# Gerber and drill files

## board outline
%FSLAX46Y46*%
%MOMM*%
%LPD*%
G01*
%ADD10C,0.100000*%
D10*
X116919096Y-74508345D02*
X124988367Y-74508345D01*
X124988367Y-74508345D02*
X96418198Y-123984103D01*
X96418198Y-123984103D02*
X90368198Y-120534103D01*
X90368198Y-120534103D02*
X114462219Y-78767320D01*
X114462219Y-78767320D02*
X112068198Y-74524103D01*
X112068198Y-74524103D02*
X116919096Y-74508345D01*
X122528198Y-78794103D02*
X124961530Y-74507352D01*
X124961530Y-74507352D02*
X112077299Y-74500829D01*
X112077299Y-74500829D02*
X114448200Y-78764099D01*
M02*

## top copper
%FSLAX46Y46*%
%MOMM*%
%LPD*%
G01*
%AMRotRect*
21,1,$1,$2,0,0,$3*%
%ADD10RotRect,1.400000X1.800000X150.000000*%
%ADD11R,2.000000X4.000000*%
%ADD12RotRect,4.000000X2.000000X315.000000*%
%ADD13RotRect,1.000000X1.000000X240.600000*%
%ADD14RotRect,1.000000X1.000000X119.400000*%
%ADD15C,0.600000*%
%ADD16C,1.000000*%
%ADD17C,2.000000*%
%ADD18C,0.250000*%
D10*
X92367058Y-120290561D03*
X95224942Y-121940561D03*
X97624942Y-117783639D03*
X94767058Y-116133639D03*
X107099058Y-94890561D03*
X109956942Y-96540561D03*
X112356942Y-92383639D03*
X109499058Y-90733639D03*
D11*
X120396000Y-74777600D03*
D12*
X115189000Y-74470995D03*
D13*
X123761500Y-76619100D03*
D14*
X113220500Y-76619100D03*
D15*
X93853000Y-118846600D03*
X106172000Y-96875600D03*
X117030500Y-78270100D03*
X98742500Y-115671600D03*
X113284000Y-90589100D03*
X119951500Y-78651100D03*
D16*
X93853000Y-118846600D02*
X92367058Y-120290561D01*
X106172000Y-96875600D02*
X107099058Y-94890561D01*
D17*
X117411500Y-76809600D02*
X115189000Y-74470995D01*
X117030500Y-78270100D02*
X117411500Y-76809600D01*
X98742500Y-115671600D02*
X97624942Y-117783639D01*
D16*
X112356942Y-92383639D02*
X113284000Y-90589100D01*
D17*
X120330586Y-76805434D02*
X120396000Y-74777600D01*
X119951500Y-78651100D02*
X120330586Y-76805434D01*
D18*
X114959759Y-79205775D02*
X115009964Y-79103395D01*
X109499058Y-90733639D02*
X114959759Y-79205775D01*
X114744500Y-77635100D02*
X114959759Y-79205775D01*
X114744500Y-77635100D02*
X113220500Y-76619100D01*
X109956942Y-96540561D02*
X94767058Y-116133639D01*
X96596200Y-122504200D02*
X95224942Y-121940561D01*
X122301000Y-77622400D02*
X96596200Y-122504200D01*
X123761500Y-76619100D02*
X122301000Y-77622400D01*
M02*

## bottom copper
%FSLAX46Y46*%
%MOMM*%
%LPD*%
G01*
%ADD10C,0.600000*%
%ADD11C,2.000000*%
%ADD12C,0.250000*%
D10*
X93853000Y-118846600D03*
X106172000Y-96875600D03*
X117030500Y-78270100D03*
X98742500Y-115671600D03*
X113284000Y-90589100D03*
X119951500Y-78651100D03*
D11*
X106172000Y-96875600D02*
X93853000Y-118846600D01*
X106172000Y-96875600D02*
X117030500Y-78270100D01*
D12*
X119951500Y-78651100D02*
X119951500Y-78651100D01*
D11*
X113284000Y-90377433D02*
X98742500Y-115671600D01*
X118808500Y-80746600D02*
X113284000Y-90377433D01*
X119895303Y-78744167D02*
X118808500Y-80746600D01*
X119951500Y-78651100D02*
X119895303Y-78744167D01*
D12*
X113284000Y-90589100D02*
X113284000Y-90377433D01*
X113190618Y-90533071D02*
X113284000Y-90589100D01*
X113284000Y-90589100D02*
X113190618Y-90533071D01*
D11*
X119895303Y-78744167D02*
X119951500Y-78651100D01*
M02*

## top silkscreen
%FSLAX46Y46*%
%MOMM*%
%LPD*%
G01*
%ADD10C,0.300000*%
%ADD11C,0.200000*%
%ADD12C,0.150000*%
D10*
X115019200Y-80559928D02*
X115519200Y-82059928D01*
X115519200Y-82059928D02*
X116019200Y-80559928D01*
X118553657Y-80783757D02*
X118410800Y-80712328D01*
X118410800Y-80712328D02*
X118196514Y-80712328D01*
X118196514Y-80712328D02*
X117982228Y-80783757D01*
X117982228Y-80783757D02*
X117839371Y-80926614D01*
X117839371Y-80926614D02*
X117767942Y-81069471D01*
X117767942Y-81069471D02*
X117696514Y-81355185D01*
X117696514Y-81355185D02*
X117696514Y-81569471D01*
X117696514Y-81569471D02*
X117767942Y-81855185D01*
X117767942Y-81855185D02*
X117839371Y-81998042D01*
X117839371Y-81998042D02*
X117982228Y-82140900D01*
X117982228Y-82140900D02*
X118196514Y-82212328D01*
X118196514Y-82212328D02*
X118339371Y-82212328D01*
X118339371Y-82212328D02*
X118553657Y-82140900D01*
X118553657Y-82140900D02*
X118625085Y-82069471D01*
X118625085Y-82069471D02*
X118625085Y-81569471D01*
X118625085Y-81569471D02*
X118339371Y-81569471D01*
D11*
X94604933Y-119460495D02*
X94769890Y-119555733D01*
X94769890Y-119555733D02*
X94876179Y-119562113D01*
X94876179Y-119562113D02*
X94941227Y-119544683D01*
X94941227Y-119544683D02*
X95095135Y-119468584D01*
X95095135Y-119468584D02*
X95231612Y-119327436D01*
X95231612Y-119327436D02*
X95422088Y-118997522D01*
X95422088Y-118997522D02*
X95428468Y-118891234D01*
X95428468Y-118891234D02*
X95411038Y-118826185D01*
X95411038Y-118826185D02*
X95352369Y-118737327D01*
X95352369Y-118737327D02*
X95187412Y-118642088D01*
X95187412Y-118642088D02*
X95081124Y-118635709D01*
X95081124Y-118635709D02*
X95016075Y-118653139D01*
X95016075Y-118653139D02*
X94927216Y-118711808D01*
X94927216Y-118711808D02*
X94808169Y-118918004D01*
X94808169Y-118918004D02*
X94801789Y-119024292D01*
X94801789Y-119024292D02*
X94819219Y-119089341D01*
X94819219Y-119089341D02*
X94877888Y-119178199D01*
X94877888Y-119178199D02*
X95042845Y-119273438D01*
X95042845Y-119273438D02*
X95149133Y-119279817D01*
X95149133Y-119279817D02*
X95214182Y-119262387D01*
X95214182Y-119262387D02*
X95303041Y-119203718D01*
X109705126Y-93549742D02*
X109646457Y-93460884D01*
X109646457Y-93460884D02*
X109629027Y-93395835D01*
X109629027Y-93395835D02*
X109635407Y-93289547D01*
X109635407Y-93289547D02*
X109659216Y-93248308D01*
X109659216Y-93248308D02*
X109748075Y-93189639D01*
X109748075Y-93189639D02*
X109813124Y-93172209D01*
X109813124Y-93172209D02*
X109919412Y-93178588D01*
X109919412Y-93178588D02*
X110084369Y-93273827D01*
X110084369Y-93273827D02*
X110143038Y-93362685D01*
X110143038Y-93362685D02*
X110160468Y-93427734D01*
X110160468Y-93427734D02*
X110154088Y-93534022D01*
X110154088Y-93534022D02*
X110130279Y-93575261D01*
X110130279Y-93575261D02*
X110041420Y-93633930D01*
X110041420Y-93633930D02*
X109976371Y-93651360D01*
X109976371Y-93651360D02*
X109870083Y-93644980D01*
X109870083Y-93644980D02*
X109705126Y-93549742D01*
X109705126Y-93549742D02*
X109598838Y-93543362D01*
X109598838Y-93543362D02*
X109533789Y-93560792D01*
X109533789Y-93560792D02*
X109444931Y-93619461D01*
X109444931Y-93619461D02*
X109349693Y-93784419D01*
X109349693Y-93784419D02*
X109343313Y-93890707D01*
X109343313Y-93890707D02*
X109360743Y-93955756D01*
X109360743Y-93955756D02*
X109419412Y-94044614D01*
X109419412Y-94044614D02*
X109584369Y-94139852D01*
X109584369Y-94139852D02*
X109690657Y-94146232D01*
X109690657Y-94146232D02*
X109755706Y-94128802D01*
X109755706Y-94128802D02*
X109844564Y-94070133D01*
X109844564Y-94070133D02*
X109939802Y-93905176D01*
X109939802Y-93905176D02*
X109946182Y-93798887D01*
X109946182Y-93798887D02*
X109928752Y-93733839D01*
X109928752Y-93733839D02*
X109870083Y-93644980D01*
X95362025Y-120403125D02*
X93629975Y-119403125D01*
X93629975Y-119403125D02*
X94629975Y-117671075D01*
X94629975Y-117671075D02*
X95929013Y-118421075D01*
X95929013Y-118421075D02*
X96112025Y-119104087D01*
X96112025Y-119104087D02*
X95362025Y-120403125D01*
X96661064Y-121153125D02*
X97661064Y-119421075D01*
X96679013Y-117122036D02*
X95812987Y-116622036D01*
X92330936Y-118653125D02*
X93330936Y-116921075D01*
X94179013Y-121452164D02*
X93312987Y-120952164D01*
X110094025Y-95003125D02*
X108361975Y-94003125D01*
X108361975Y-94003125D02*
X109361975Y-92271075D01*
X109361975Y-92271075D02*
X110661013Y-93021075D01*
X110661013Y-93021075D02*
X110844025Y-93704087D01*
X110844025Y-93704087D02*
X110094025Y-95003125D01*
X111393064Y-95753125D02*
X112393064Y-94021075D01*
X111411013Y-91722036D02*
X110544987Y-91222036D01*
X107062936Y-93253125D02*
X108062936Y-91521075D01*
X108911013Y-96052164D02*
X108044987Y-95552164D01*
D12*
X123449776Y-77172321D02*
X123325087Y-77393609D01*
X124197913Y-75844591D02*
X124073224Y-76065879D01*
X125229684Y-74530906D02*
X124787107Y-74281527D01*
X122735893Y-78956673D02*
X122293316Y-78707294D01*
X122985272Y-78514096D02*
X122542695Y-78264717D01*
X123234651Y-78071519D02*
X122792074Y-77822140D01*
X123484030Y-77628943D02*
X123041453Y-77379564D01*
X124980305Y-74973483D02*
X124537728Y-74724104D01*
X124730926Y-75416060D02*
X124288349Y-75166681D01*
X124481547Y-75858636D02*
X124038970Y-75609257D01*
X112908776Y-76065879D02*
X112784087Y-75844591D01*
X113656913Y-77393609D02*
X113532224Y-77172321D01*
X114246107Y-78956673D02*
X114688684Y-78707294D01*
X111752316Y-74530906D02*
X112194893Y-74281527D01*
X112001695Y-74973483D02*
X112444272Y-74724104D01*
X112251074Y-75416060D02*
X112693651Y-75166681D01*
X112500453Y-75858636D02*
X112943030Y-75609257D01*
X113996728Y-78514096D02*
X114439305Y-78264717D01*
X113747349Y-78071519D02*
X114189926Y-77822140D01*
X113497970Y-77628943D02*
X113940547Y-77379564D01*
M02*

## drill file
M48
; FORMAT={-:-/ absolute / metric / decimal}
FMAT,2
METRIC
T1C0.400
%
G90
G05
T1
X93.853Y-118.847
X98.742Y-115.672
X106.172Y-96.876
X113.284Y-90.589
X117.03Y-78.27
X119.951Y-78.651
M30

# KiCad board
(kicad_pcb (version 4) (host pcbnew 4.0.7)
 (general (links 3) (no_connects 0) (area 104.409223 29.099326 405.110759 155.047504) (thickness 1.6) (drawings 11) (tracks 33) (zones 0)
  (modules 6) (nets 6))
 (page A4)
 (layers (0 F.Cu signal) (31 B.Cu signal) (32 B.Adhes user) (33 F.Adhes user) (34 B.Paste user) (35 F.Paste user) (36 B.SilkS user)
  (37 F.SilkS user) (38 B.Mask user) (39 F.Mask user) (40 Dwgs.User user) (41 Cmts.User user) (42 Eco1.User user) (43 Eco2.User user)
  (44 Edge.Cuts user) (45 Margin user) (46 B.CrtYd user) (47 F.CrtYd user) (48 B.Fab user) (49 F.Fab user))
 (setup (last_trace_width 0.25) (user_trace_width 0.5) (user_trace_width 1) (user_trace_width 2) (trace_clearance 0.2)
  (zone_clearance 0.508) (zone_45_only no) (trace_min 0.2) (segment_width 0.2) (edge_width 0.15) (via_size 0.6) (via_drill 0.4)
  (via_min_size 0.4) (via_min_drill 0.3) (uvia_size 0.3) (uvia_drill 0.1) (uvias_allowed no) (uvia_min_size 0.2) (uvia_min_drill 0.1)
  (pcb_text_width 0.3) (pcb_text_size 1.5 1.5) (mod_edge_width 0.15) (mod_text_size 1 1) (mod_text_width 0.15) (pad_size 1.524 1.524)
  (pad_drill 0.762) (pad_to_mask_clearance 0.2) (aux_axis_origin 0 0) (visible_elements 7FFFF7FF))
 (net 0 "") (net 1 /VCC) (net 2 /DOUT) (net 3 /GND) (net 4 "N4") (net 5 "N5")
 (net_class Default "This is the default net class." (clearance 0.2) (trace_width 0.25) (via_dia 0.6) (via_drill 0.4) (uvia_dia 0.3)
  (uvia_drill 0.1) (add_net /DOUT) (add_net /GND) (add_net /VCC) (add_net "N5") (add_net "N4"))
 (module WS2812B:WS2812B (layer F.Cu) (at 94.996 119.0371 150)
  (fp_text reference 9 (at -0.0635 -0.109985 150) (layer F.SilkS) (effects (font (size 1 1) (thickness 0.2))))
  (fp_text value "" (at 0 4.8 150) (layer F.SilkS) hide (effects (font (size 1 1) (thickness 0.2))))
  (fp_line (start -1 -1) (end 1 -1) (layer F.SilkS) (width 0.2)) (fp_line (start 1 -1) (end 1 1) (layer F.SilkS) (width 0.2))
  (fp_line (start 1 1) (end -0.5 1) (layer F.SilkS) (width 0.2))
  (fp_line (start -0.5 1) (end -1 0.5) (layer F.SilkS) (width 0.2))
  (fp_line (start -1 0.5) (end -1 -1) (layer F.SilkS) (width 0.2))
  (fp_line (start -2.5 -1) (end -2.5 1) (layer F.SilkS) (width 0.2))
  (fp_line (start -0.5 2.5) (end 0.5 2.5) (layer F.SilkS) (width 0.2))
  (fp_line (start 2.5 -1) (end 2.5 1) (layer F.SilkS) (width 0.2))
  (fp_line (start -0.5 -2.5) (end 0.5 -2.5) (layer F.SilkS) (width 0.2))
  (pad 1 smd rect (at 1.65 -2.4 150) (size 1.4 1.8) (layers F.Cu F.Paste F.Mask) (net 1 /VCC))
  (pad 2 smd rect (at -1.65 -2.4 150) (size 1.4 1.8) (layers F.Cu F.Paste F.Mask) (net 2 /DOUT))
  (pad 3 smd rect (at -1.65 2.4 150) (size 1.4 1.8) (layers F.Cu F.Paste F.Mask) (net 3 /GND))
  (pad 4 smd rect (at 1.65 2.4 150) (size 1.4 1.8) (layers F.Cu F.Paste F.Mask) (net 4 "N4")))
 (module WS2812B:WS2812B (layer F.Cu) (at 109.728 93.6371 150)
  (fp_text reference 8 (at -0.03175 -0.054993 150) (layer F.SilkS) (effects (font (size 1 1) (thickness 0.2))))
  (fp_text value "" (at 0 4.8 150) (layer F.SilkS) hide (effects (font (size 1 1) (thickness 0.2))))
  (fp_line (start -1 -1) (end 1 -1) (layer F.SilkS) (width 0.2)) (fp_line (start 1 -1) (end 1 1) (layer F.SilkS) (width 0.2))
  (fp_line (start 1 1) (end -0.5 1) (layer F.SilkS) (width 0.2))
  (fp_line (start -0.5 1) (end -1 0.5) (layer F.SilkS) (width 0.2))
  (fp_line (start -1 0.5) (end -1 -1) (layer F.SilkS) (width 0.2))
  (fp_line (start -2.5 -1) (end -2.5 1) (layer F.SilkS) (width 0.2))
  (fp_line (start -0.5 2.5) (end 0.5 2.5) (layer F.SilkS) (width 0.2))
  (fp_line (start 2.5 -1) (end 2.5 1) (layer F.SilkS) (width 0.2))
  (fp_line (start -0.5 -2.5) (end 0.5 -2.5) (layer F.SilkS) (width 0.2))
  (pad 1 smd rect (at 1.65 -2.4 150) (size 1.4 1.8) (layers F.Cu F.Paste F.Mask) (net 1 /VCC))
  (pad 2 smd rect (at -1.65 -2.4 150) (size 1.4 1.8) (layers F.Cu F.Paste F.Mask) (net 4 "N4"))
  (pad 3 smd rect (at -1.65 2.4 150) (size 1.4 1.8) (layers F.Cu F.Paste F.Mask) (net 3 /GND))
  (pad 4 smd rect (at 1.65 2.4 150) (size 1.4 1.8) (layers F.Cu F.Paste F.Mask) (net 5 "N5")))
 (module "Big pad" (layer F.Cu) (at 120.523 74.6506 90)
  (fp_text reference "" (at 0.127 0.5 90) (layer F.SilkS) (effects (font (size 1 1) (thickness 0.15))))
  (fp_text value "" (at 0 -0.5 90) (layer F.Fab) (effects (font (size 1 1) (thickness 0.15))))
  (pad 1 smd rect (at -0.127 -0.127 90) (size 4 2) (layers F.Cu F.Paste F.Mask)))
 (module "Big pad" (layer F.Cu) (at 115.189 74.6506 315)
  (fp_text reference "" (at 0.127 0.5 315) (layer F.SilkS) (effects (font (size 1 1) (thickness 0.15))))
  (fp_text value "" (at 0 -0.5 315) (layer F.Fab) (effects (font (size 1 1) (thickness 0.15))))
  (pad 1 smd rect (at -0.127 -0.127 315) (size 4 2) (layers F.Cu F.Paste F.Mask)))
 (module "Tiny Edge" (layer F.Cu) (at 123.7615 76.6191 240.6)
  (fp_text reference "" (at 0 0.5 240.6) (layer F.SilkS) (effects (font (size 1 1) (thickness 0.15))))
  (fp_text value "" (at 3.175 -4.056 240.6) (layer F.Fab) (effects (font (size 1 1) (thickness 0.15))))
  (fp_line (start 0.635 0) (end 0.889 0) (layer F.SilkS) (width 0.15))
  (fp_line (start -0.889 0) (end -0.635 0) (layer F.SilkS) (width 0.15))
  (fp_line (start -2.54 -0.254) (end -2.54 0.254) (layer F.SilkS) (width 0.15))
  (fp_line (start 2.54 -0.254) (end 2.54 0.254) (layer F.SilkS) (width 0.15))
  (fp_line (start 2.032 -0.254) (end 2.032 0.254) (layer F.SilkS) (width 0.15))
  (fp_line (start 1.524 -0.254) (end 1.524 0.254) (layer F.SilkS) (width 0.15))
  (fp_line (start 1.016 -0.254) (end 1.016 0.254) (layer F.SilkS) (width 0.15))
  (fp_line (start -2.032 -0.254) (end -2.032 0.254) (layer F.SilkS) (width 0.15))
  (fp_line (start -1.524 -0.254) (end -1.524 0.254) (layer F.SilkS) (width 0.15))
  (fp_line (start -1.016 -0.254) (end -1.016 0.254) (layer F.SilkS) (width 0.15))
  (pad 1 smd rect (at 0 0 240.6) (size 1 1) (layers F.Cu F.Paste F.Mask)))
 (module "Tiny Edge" (layer F.Cu) (at 113.2205 76.6191 119.4)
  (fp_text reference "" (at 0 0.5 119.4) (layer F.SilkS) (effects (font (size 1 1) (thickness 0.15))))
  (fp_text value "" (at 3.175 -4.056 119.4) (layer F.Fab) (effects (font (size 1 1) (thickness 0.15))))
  (fp_line (start 0.635 0) (end 0.889 0) (layer F.SilkS) (width 0.15))
  (fp_line (start -0.889 0) (end -0.635 0) (layer F.SilkS) (width 0.15))
  (fp_line (start -2.54 -0.254) (end -2.54 0.254) (layer F.SilkS) (width 0.15))
  (fp_line (start 2.54 -0.254) (end 2.54 0.254) (layer F.SilkS) (width 0.15))
  (fp_line (start 2.032 -0.254) (end 2.032 0.254) (layer F.SilkS) (width 0.15))
  (fp_line (start 1.524 -0.254) (end 1.524 0.254) (layer F.SilkS) (width 0.15))
  (fp_line (start 1.016 -0.254) (end 1.016 0.254) (layer F.SilkS) (width 0.15))
  (fp_line (start -2.032 -0.254) (end -2.032 0.254) (layer F.SilkS) (width 0.15))
  (fp_line (start -1.524 -0.254) (end -1.524 0.254) (layer F.SilkS) (width 0.15))
  (fp_line (start -1.016 -0.254) (end -1.016 0.254) (layer F.SilkS) (width 0.15))
  (pad 1 smd rect (at 0 0 119.4) (size 1 1) (layers F.Cu F.Paste F.Mask)))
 (gr_line (start 116.919096 74.508345) (end 124.988367 74.508345) (layer Edge.Cuts) (width 0.1))
 (gr_line (start 124.988367 74.508345) (end 96.418198 123.984103) (layer Edge.Cuts) (width 0.1))
 (gr_line (start 96.418198 123.984103) (end 90.368198 120.534103) (layer Edge.Cuts) (width 0.1))
 (gr_line (start 90.368198 120.534103) (end 114.462219 78.76732) (layer Edge.Cuts) (width 0.1))
 (gr_line (start 114.462219 78.76732) (end 112.068198 74.524103) (layer Edge.Cuts) (width 0.1))
 (gr_line (start 112.068198 74.524103) (end 116.919096 74.508345) (layer Edge.Cuts) (width 0.1))
 (gr_line (start 122.528198 78.794103) (end 124.96153 74.507352) (layer Edge.Cuts) (width 0.1))
 (gr_line (start 124.96153 74.507352) (end 112.077299 74.500829) (layer Edge.Cuts) (width 0.1))
 (gr_line (start 112.077299 74.500829) (end 114.4482 78.764099) (layer Edge.Cuts) (width 0.1))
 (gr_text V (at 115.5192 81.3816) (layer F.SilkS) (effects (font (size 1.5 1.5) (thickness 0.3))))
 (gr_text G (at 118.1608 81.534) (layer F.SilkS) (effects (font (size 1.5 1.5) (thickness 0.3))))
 (segment (start 106.172 96.8756) (end 93.853 118.8466) (width 2) (layer B.Cu) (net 1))
 (via (at 93.853 118.8466) (size 0.6) (drill 0.4) (layers F.Cu B.Cu) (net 1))
 (segment (start 93.853 118.8466) (end 92.367058 120.290561) (width 1) (layer F.Cu) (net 1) (status 20))
 (segment (start 106.172 96.8756) (end 107.099058 94.890561) (width 1) (layer F.Cu) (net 1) (status 20))
 (via (at 106.172 96.8756) (size 0.6) (drill 0.4) (layers F.Cu B.Cu) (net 1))
 (segment (start 106.172 96.8756) (end 117.0305 78.2701) (width 2) (layer B.Cu) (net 1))
 (segment (start 117.4115 76.8096) (end 115.189 74.470995) (width 2) (layer F.Cu) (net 1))
 (segment (start 117.0305 78.2701) (end 117.4115 76.8096) (width 2) (layer F.Cu) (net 1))
 (via (at 117.0305 78.2701) (size 0.6) (drill 0.4) (layers F.Cu B.Cu) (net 1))
 (segment (start 119.9515 78.6511) (end 119.9515 78.6511) (width 0.25) (layer B.Cu) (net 3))
 (via (at 98.7425 115.6716) (size 0.6) (drill 0.4) (layers F.Cu B.Cu) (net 3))
 (segment (start 98.7425 115.6716) (end 97.624942 117.783639) (width 2) (layer F.Cu) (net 3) (status 20))
 (segment (start 113.284 90.377433) (end 98.7425 115.6716) (width 2) (layer B.Cu) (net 3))
 (segment (start 118.8085 80.7466) (end 113.284 90.377433) (width 2) (layer B.Cu) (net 3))
 (segment (start 119.895303 78.744167) (end 118.8085 80.7466) (width 2) (layer B.Cu) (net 3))
 (segment (start 119.9515 78.6511) (end 119.895303 78.744167) (width 2) (layer B.Cu) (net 3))
 (segment (start 113.284 90.5891) (end 113.284 90.377433) (width 0.25) (layer B.Cu) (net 3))
 (segment (start 113.190618 90.533071) (end 113.284 90.5891) (width 0.25) (layer B.Cu) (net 3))
 (segment (start 113.284 90.5891) (end 113.190618 90.533071) (width 0.25) (layer B.Cu) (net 3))
 (via (at 113.284 90.5891) (size 0.6) (drill 0.4) (layers F.Cu B.Cu) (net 3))
 (segment (start 112.356942 92.383639) (end 113.284 90.5891) (width 1) (layer F.Cu) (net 3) (status 10))
 (segment (start 120.330586 76.805434) (end 120.396 74.7776) (width 2) (layer F.Cu) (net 3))
 (segment (start 119.9515 78.6511) (end 120.330586 76.805434) (width 2) (layer F.Cu) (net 3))
 (via (at 119.9515 78.6511) (size 0.6) (drill 0.4) (layers F.Cu B.Cu) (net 3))
 (segment (start 119.895303 78.744167) (end 119.9515 78.6511) (width 2) (layer B.Cu) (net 3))
 (segment (start 114.959759 79.205775) (end 115.009964 79.103395) (width 0.25) (layer F.Cu) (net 5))
 (segment (start 109.499058 90.733639) (end 114.959759 79.205775) (width 0.25) (layer F.Cu) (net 5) (status 10))
 (segment (start 114.7445 77.6351) (end 114.959759 79.205775) (width 0.25) (layer F.Cu) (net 5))
 (segment (start 114.7445 77.6351) (end 113.2205 76.6191) (width 0.25) (layer F.Cu) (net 5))
 (segment (start 109.956942 96.540561) (end 94.767058 116.133639) (width 0.25) (layer F.Cu) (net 4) (status 20))
 (segment (start 96.5962 122.5042) (end 95.224942 121.940561) (width 0.25) (layer F.Cu) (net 2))
 (segment (start 122.301 77.6224) (end 96.5962 122.5042) (width 0.25) (layer F.Cu) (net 2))
 (segment (start 123.7615 76.6191) (end 122.301 77.6224) (width 0.25) (layer F.Cu) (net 2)))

